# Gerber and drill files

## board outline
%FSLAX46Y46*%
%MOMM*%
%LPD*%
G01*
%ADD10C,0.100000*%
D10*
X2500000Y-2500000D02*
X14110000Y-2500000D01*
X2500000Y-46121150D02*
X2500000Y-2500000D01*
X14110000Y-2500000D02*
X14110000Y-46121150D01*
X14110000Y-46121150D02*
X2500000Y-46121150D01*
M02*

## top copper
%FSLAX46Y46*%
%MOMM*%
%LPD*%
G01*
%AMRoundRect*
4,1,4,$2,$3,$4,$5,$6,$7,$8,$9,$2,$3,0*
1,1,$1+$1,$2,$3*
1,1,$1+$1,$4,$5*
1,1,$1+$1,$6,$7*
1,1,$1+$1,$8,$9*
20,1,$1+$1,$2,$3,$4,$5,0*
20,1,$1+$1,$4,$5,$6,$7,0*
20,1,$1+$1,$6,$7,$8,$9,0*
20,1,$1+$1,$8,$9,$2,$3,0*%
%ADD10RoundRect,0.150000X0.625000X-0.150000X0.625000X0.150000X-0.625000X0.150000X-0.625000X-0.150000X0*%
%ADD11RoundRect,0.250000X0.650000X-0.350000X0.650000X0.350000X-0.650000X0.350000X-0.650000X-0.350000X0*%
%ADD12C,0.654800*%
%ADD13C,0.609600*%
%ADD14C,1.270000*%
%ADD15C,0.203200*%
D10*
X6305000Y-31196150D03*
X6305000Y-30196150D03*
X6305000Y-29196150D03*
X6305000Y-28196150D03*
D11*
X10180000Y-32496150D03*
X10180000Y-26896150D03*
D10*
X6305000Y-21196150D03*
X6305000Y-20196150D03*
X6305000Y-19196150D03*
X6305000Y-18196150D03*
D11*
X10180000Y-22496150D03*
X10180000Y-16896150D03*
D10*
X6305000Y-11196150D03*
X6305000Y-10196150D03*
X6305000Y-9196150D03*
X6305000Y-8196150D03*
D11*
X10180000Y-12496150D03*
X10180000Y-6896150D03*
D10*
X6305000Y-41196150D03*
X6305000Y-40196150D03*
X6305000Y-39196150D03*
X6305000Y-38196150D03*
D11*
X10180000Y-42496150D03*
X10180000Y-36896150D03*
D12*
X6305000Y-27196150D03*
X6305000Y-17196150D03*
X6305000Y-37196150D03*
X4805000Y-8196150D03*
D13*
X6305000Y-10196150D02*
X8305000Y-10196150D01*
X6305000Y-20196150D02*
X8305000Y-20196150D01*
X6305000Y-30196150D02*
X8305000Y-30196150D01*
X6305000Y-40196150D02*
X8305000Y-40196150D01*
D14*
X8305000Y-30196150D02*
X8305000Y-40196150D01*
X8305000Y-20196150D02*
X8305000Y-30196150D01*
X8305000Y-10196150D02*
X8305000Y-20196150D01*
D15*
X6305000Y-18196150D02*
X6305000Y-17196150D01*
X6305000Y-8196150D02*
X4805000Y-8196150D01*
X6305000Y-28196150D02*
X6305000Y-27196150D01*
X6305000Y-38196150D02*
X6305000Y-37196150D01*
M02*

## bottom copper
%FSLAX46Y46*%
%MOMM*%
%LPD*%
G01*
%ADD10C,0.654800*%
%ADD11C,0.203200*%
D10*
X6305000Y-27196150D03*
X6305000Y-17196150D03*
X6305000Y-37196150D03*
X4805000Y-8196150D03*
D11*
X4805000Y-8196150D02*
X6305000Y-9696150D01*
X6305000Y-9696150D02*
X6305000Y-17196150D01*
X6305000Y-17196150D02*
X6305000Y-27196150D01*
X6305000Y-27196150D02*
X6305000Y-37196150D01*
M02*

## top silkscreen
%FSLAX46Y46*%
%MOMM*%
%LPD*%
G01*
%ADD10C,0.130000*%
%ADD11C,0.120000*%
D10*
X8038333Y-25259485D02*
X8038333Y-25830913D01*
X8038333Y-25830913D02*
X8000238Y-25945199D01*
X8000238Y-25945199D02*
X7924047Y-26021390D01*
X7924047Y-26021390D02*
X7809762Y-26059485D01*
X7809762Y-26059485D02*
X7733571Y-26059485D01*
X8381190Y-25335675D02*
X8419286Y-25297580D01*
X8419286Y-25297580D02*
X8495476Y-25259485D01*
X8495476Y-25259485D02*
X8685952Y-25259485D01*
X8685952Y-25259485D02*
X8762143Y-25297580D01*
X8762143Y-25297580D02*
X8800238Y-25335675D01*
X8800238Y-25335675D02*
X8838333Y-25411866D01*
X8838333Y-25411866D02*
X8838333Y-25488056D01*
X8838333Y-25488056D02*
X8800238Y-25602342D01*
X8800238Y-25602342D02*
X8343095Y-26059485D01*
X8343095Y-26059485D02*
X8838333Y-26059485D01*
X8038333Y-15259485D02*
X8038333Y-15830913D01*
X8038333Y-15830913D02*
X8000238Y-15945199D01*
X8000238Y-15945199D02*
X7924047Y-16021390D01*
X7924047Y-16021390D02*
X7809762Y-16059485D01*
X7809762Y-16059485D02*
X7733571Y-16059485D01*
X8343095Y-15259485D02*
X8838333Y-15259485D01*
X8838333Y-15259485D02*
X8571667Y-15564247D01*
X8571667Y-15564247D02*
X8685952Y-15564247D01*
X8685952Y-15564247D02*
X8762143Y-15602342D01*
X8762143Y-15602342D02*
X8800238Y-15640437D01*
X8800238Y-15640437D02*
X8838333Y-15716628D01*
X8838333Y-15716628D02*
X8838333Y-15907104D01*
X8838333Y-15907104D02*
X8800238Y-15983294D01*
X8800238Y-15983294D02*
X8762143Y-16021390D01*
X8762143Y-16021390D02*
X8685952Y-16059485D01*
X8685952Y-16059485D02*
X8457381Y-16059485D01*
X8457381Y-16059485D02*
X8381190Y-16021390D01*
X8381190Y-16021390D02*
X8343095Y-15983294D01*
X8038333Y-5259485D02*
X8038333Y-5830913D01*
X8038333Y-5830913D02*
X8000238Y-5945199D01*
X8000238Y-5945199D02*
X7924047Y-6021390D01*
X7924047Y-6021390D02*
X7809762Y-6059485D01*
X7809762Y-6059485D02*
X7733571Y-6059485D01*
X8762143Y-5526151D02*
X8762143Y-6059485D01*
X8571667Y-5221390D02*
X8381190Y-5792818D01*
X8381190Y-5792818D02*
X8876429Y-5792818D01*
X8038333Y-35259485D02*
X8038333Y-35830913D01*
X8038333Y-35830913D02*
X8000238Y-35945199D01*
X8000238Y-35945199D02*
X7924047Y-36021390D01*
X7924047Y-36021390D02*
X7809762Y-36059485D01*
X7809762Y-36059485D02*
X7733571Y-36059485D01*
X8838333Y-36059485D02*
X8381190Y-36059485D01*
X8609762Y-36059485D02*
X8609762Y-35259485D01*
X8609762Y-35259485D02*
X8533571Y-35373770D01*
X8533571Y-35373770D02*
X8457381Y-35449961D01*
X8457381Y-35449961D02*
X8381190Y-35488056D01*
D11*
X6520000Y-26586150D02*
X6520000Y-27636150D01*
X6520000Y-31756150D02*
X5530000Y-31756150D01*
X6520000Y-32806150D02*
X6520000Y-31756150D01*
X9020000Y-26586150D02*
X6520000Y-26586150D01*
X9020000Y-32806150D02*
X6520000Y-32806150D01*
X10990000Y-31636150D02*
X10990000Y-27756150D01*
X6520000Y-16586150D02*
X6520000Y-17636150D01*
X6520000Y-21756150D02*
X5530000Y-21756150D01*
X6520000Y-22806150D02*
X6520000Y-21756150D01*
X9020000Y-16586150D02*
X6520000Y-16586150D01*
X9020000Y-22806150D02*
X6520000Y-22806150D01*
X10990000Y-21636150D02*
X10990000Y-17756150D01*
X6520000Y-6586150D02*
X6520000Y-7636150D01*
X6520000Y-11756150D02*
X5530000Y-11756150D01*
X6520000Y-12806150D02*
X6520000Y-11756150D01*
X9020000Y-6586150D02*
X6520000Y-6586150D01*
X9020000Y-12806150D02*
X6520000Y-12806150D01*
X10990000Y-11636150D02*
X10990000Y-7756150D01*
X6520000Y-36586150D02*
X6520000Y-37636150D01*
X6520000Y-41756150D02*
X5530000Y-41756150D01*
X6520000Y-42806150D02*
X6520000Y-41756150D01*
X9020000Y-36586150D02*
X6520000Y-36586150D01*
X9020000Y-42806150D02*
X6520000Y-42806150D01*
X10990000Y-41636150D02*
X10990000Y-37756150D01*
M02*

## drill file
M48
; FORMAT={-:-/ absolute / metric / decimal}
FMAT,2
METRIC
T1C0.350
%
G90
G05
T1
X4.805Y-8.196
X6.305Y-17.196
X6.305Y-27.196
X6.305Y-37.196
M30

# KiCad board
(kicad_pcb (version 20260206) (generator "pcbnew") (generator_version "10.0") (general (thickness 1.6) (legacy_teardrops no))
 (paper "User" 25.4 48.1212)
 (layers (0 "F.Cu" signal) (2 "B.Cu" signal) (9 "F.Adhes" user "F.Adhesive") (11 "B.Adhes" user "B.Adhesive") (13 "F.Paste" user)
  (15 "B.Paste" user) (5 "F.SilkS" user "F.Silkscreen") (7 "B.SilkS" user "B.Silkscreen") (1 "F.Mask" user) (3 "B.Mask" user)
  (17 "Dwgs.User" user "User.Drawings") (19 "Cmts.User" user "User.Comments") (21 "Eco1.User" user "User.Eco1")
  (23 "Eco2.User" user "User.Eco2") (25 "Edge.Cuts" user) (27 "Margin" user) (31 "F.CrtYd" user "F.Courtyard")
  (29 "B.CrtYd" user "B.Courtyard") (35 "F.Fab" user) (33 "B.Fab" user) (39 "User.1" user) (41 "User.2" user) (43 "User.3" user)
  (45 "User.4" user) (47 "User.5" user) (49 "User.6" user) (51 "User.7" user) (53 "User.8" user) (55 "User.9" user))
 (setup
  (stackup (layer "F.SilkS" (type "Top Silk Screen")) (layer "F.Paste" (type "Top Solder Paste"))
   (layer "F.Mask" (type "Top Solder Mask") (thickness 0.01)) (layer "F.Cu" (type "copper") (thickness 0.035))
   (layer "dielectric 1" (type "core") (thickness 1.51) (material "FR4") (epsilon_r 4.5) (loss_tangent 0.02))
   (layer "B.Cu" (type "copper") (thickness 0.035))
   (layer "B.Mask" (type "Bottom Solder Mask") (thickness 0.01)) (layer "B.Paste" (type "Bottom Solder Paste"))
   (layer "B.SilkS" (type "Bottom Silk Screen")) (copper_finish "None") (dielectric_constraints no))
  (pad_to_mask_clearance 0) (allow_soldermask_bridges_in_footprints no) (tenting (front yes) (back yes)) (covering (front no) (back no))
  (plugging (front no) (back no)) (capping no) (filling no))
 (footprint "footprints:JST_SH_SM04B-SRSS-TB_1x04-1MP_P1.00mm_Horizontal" (layer "F.Cu") (at 8.305 29.69615 90)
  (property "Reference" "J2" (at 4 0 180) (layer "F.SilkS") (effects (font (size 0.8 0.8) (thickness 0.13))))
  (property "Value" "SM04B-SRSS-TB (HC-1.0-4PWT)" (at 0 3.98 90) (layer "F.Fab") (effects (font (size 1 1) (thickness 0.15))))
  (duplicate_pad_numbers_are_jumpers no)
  (fp_line (start 3.11 -1.785) (end 2.06 -1.785) (stroke (width 0.12) (type solid)) (layer "F.SilkS"))
  (fp_line (start -2.06 -1.785) (end -2.06 -2.775) (stroke (width 0.12) (type solid)) (layer "F.SilkS"))
  (fp_line (start -3.11 -1.785) (end -2.06 -1.785) (stroke (width 0.12) (type solid)) (layer "F.SilkS"))
  (fp_line (start 3.11 0.715) (end 3.11 -1.785) (stroke (width 0.12) (type solid)) (layer "F.SilkS"))
  (fp_line (start -3.11 0.715) (end -3.11 -1.785) (stroke (width 0.12) (type solid)) (layer "F.SilkS"))
  (fp_line (start -1.94 2.685) (end 1.94 2.685) (stroke (width 0.12) (type solid)) (layer "F.SilkS"))
  (pad "1" smd roundrect (at -1.5 -2 90) (size 0.6 1.55) (layers "F.Cu" "F.Mask" "F.Paste") (roundrect_rratio 0.25) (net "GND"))
  (pad "2" smd roundrect (at -0.5 -2 90) (size 0.6 1.55) (layers "F.Cu" "F.Mask" "F.Paste") (roundrect_rratio 0.25) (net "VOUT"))
  (pad "3" smd roundrect (at 0.5 -2 90) (size 0.6 1.55) (layers "F.Cu" "F.Mask" "F.Paste") (roundrect_rratio 0.25) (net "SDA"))
  (pad "4" smd roundrect (at 1.5 -2 90) (size 0.6 1.55) (layers "F.Cu" "F.Mask" "F.Paste") (roundrect_rratio 0.25) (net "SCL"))
  (pad "MP" smd roundrect (at -2.8 1.875 90) (size 1.2 1.8) (layers "F.Cu" "F.Mask" "F.Paste") (roundrect_rratio 0.208333) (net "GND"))
  (pad "MP" smd roundrect (at 2.8 1.875 90) (size 1.2 1.8) (layers "F.Cu" "F.Mask" "F.Paste") (roundrect_rratio 0.208333) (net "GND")))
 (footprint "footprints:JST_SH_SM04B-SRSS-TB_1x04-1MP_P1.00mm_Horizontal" (layer "F.Cu") (at 8.305 19.69615 90)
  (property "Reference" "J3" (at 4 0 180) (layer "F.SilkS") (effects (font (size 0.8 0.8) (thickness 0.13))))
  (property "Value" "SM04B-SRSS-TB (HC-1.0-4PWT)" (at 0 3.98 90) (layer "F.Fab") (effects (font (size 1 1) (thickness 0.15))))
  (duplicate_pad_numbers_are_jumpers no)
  (fp_line (start 3.11 -1.785) (end 2.06 -1.785) (stroke (width 0.12) (type solid)) (layer "F.SilkS"))
  (fp_line (start -2.06 -1.785) (end -2.06 -2.775) (stroke (width 0.12) (type solid)) (layer "F.SilkS"))
  (fp_line (start -3.11 -1.785) (end -2.06 -1.785) (stroke (width 0.12) (type solid)) (layer "F.SilkS"))
  (fp_line (start 3.11 0.715) (end 3.11 -1.785) (stroke (width 0.12) (type solid)) (layer "F.SilkS"))
  (fp_line (start -3.11 0.715) (end -3.11 -1.785) (stroke (width 0.12) (type solid)) (layer "F.SilkS"))
  (fp_line (start -1.94 2.685) (end 1.94 2.685) (stroke (width 0.12) (type solid)) (layer "F.SilkS"))
  (pad "1" smd roundrect (at -1.5 -2 90) (size 0.6 1.55) (layers "F.Cu" "F.Mask" "F.Paste") (roundrect_rratio 0.25) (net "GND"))
  (pad "2" smd roundrect (at -0.5 -2 90) (size 0.6 1.55) (layers "F.Cu" "F.Mask" "F.Paste") (roundrect_rratio 0.25) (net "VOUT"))
  (pad "3" smd roundrect (at 0.5 -2 90) (size 0.6 1.55) (layers "F.Cu" "F.Mask" "F.Paste") (roundrect_rratio 0.25) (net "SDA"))
  (pad "4" smd roundrect (at 1.5 -2 90) (size 0.6 1.55) (layers "F.Cu" "F.Mask" "F.Paste") (roundrect_rratio 0.25) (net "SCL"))
  (pad "MP" smd roundrect (at -2.8 1.875 90) (size 1.2 1.8) (layers "F.Cu" "F.Mask" "F.Paste") (roundrect_rratio 0.208333) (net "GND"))
  (pad "MP" smd roundrect (at 2.8 1.875 90) (size 1.2 1.8) (layers "F.Cu" "F.Mask" "F.Paste") (roundrect_rratio 0.208333) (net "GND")))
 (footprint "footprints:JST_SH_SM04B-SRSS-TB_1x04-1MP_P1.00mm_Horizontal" (layer "F.Cu") (at 8.305 9.69615 90)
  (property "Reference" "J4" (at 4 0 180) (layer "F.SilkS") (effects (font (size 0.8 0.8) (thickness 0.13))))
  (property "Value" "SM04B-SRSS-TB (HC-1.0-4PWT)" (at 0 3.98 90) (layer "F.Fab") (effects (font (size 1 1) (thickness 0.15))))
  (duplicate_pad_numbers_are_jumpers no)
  (fp_line (start 3.11 -1.785) (end 2.06 -1.785) (stroke (width 0.12) (type solid)) (layer "F.SilkS"))
  (fp_line (start -2.06 -1.785) (end -2.06 -2.775) (stroke (width 0.12) (type solid)) (layer "F.SilkS"))
  (fp_line (start -3.11 -1.785) (end -2.06 -1.785) (stroke (width 0.12) (type solid)) (layer "F.SilkS"))
  (fp_line (start 3.11 0.715) (end 3.11 -1.785) (stroke (width 0.12) (type solid)) (layer "F.SilkS"))
  (fp_line (start -3.11 0.715) (end -3.11 -1.785) (stroke (width 0.12) (type solid)) (layer "F.SilkS"))
  (fp_line (start -1.94 2.685) (end 1.94 2.685) (stroke (width 0.12) (type solid)) (layer "F.SilkS"))
  (pad "1" smd roundrect (at -1.5 -2 90) (size 0.6 1.55) (layers "F.Cu" "F.Mask" "F.Paste") (roundrect_rratio 0.25) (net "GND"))
  (pad "2" smd roundrect (at -0.5 -2 90) (size 0.6 1.55) (layers "F.Cu" "F.Mask" "F.Paste") (roundrect_rratio 0.25) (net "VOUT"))
  (pad "3" smd roundrect (at 0.5 -2 90) (size 0.6 1.55) (layers "F.Cu" "F.Mask" "F.Paste") (roundrect_rratio 0.25) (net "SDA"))
  (pad "4" smd roundrect (at 1.5 -2 90) (size 0.6 1.55) (layers "F.Cu" "F.Mask" "F.Paste") (roundrect_rratio 0.25) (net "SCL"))
  (pad "MP" smd roundrect (at -2.8 1.875 90) (size 1.2 1.8) (layers "F.Cu" "F.Mask" "F.Paste") (roundrect_rratio 0.208333) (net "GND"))
  (pad "MP" smd roundrect (at 2.8 1.875 90) (size 1.2 1.8) (layers "F.Cu" "F.Mask" "F.Paste") (roundrect_rratio 0.208333) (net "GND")))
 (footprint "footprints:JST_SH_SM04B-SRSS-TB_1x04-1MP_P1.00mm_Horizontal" (layer "F.Cu") (at 8.305 39.69615 90)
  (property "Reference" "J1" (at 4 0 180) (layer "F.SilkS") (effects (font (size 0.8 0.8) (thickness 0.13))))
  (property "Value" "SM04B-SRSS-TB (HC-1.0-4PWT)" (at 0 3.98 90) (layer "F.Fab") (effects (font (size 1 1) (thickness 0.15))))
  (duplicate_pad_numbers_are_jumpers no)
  (fp_line (start 3.11 -1.785) (end 2.06 -1.785) (stroke (width 0.12) (type solid)) (layer "F.SilkS"))
  (fp_line (start -2.06 -1.785) (end -2.06 -2.775) (stroke (width 0.12) (type solid)) (layer "F.SilkS"))
  (fp_line (start -3.11 -1.785) (end -2.06 -1.785) (stroke (width 0.12) (type solid)) (layer "F.SilkS"))
  (fp_line (start 3.11 0.715) (end 3.11 -1.785) (stroke (width 0.12) (type solid)) (layer "F.SilkS"))
  (fp_line (start -3.11 0.715) (end -3.11 -1.785) (stroke (width 0.12) (type solid)) (layer "F.SilkS"))
  (fp_line (start -1.94 2.685) (end 1.94 2.685) (stroke (width 0.12) (type solid)) (layer "F.SilkS"))
  (pad "1" smd roundrect (at -1.5 -2 90) (size 0.6 1.55) (layers "F.Cu" "F.Mask" "F.Paste") (roundrect_rratio 0.25) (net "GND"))
  (pad "2" smd roundrect (at -0.5 -2 90) (size 0.6 1.55) (layers "F.Cu" "F.Mask" "F.Paste") (roundrect_rratio 0.25) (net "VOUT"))
  (pad "3" smd roundrect (at 0.5 -2 90) (size 0.6 1.55) (layers "F.Cu" "F.Mask" "F.Paste") (roundrect_rratio 0.25) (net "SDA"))
  (pad "4" smd roundrect (at 1.5 -2 90) (size 0.6 1.55) (layers "F.Cu" "F.Mask" "F.Paste") (roundrect_rratio 0.25) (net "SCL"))
  (pad "MP" smd roundrect (at -2.8 1.875 90) (size 1.2 1.8) (layers "F.Cu" "F.Mask" "F.Paste") (roundrect_rratio 0.208333) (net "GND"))
  (pad "MP" smd roundrect (at 2.8 1.875 90) (size 1.2 1.8) (layers "F.Cu" "F.Mask" "F.Paste") (roundrect_rratio 0.208333) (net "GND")))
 (gr_line (start 2.5 2.5) (end 14.11 2.5) (stroke (width 0.1) (type default)) (layer "Edge.Cuts"))
 (gr_line (start 2.5 46.12115) (end 2.5 2.5) (stroke (width 0.1) (type default)) (layer "Edge.Cuts"))
 (gr_line (start 14.11 2.5) (end 14.11 46.12115) (stroke (width 0.1) (type default)) (layer "Edge.Cuts"))
 (gr_line (start 14.11 46.12115) (end 2.5 46.12115) (stroke (width 0.1) (type default)) (layer "Edge.Cuts"))
 (segment (start 6.305 10.19615) (end 8.305 10.19615) (width 0.6096) (layer "F.Cu") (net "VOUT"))
 (segment (start 6.305 20.19615) (end 8.305 20.19615) (width 0.6096) (layer "F.Cu") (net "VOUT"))
 (segment (start 6.305 30.19615) (end 8.305 30.19615) (width 0.6096) (layer "F.Cu") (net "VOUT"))
 (segment (start 6.305 40.19615) (end 8.305 40.19615) (width 0.6096) (layer "F.Cu") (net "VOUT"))
 (segment (start 8.305 30.19615) (end 8.305 40.19615) (width 1.27) (layer "F.Cu") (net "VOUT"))
 (segment (start 8.305 20.19615) (end 8.305 30.19615) (width 1.27) (layer "F.Cu") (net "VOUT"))
 (segment (start 8.305 10.19615) (end 8.305 20.19615) (width 1.27) (layer "F.Cu") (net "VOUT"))
 (segment (start 6.305 18.19615) (end 6.305 17.19615) (width 0.2032) (layer "F.Cu") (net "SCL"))
 (segment (start 6.305 8.19615) (end 4.805 8.19615) (width 0.2032) (layer "F.Cu") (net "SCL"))
 (segment (start 6.305 28.19615) (end 6.305 27.19615) (width 0.2032) (layer "F.Cu") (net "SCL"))
 (segment (start 6.305 38.19615) (end 6.305 37.19615) (width 0.2032) (layer "F.Cu") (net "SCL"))
 (via (at 6.305 27.19615) (size 0.6548) (drill 0.35) (layers "F.Cu" "B.Cu") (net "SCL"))
 (via (at 6.305 17.19615) (size 0.6548) (drill 0.35) (layers "F.Cu" "B.Cu") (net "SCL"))
 (via (at 6.305 37.19615) (size 0.6548) (drill 0.35) (layers "F.Cu" "B.Cu") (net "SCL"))
 (via (at 4.805 8.19615) (size 0.6548) (drill 0.35) (layers "F.Cu" "B.Cu") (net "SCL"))
 (segment (start 4.805 8.19615) (end 6.305 9.69615) (width 0.2032) (layer "B.Cu") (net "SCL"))
 (segment (start 6.305 9.69615) (end 6.305 17.19615) (width 0.2032) (layer "B.Cu") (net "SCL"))
 (segment (start 6.305 17.19615) (end 6.305 27.19615) (width 0.2032) (layer "B.Cu") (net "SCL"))
 (segment (start 6.305 27.19615) (end 6.305 37.19615) (width 0.2032) (layer "B.Cu") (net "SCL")))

